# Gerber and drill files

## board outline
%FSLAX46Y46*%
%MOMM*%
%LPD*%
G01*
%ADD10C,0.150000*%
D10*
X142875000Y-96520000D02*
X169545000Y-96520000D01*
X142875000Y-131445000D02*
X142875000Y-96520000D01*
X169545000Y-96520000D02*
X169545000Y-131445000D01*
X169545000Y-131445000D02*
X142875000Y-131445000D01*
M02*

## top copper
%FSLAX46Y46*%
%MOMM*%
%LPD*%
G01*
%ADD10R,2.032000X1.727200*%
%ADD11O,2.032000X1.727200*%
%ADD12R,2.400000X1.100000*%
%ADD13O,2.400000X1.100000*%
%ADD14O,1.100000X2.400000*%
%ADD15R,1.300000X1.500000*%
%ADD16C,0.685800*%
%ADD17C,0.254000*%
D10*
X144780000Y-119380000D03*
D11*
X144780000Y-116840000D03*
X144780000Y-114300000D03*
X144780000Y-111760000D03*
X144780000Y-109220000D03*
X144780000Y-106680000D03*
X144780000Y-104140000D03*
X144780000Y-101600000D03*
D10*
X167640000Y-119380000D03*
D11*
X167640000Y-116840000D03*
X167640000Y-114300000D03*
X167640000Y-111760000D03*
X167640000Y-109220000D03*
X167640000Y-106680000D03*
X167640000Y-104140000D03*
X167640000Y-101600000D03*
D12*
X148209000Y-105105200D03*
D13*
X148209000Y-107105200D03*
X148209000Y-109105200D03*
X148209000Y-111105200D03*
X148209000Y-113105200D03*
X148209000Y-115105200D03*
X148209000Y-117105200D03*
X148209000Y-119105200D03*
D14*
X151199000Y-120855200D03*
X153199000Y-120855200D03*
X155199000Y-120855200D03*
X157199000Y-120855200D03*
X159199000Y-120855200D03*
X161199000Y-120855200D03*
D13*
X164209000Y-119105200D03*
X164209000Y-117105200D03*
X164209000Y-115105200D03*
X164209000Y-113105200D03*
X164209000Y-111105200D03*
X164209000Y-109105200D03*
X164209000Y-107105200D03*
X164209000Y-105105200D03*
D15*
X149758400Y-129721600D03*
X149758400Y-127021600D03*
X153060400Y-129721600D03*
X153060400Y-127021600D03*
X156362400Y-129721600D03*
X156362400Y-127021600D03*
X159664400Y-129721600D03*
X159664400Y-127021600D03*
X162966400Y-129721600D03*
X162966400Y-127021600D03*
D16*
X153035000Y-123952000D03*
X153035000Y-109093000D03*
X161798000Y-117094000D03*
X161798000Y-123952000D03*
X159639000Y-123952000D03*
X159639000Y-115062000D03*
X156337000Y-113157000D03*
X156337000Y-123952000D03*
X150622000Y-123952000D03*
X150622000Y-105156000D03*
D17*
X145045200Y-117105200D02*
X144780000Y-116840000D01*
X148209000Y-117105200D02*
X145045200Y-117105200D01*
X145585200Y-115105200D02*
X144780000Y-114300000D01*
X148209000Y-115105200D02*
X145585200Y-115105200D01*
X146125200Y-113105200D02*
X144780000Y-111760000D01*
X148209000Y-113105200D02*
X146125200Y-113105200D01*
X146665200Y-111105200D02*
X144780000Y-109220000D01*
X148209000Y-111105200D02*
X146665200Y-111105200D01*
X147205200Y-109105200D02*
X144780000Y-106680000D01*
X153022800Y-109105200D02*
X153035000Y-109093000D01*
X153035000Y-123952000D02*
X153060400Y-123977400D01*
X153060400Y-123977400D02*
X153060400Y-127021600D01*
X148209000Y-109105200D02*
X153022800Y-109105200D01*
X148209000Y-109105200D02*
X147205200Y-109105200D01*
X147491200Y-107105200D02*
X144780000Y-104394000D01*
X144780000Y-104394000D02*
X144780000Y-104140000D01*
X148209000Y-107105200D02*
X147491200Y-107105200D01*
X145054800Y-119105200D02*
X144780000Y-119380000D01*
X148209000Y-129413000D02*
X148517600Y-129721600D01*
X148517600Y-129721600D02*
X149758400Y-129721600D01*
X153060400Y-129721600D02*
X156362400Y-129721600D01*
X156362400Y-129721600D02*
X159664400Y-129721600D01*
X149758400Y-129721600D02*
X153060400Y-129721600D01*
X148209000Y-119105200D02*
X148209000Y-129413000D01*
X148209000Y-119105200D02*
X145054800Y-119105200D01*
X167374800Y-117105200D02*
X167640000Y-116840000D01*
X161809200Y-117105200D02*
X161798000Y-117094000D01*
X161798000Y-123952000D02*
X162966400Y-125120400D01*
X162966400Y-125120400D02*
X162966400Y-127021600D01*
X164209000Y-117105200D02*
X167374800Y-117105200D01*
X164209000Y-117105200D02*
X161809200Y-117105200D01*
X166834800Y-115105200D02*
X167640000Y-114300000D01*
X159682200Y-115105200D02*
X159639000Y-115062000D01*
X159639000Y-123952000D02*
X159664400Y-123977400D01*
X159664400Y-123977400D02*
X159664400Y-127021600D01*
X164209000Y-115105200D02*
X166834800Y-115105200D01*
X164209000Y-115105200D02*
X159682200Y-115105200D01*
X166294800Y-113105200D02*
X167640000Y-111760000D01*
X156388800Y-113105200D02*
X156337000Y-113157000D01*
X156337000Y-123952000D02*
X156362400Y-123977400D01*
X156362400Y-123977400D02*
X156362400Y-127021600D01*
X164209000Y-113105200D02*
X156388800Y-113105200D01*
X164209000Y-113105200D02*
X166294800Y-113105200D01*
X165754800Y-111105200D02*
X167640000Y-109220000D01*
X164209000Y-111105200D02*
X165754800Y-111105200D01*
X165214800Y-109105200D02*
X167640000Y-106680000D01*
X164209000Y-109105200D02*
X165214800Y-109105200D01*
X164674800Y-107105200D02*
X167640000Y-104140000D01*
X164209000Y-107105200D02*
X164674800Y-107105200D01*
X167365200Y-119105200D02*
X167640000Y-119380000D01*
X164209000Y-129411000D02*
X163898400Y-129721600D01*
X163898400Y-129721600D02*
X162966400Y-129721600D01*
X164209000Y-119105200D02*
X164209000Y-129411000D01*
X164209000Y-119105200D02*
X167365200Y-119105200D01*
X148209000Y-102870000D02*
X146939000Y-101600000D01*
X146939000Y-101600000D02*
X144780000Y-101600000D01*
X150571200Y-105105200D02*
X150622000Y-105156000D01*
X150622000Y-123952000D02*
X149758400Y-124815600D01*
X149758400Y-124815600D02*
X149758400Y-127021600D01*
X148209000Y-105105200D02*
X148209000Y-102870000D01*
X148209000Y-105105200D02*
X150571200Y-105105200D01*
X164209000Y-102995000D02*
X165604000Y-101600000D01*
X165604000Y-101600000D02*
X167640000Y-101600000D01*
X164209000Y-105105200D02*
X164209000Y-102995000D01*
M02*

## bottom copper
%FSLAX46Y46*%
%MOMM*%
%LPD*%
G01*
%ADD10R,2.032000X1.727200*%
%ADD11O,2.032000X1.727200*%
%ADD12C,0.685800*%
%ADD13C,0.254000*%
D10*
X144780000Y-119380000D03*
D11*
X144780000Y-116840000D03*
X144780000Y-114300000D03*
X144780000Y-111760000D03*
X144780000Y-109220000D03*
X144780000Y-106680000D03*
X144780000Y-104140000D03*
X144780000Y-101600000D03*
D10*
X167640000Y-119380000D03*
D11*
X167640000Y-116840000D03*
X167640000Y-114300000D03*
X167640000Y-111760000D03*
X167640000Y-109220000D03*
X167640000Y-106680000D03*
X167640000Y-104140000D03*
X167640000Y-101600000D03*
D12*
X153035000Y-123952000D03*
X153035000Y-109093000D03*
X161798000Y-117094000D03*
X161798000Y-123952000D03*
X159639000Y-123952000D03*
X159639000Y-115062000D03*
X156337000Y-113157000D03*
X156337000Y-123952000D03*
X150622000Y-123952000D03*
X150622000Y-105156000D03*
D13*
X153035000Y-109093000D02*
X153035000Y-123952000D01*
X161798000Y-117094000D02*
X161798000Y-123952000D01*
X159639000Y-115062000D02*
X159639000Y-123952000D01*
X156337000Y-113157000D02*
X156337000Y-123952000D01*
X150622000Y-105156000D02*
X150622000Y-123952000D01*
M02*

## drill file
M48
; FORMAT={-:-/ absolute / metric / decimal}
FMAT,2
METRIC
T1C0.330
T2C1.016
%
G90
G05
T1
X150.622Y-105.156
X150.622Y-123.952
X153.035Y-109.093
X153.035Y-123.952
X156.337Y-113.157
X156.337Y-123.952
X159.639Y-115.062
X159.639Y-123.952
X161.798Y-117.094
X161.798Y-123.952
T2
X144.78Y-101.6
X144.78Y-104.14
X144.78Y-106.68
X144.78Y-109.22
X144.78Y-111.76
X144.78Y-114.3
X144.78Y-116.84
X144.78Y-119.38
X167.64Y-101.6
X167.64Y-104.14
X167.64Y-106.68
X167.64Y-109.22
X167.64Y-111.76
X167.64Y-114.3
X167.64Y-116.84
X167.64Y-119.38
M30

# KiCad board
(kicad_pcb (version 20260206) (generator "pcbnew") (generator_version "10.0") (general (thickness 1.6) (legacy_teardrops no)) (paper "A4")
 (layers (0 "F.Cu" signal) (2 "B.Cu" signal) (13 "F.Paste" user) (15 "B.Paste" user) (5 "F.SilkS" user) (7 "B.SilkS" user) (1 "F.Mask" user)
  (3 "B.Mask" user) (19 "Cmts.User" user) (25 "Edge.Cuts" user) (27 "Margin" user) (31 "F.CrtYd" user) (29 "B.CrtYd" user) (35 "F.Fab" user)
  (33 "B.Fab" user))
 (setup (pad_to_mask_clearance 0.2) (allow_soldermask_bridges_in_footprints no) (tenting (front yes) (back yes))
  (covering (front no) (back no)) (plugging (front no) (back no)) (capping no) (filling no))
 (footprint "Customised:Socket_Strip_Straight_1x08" (layer "F.Cu") (at 144.78 119.38 90)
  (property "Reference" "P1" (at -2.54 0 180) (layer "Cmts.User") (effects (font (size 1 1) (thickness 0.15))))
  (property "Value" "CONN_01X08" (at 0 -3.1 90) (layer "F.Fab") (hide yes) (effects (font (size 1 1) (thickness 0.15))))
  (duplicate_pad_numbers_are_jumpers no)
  (pad "1" thru_hole rect (at 0 0 90) (size 1.7272 2.032) (drill 1.016) (layers "*.Cu" "*.Mask") (remove_unused_layers no) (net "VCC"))
  (pad "2" thru_hole oval (at 2.54 0 90) (size 1.7272 2.032) (drill 1.016) (layers "*.Cu" "*.Mask") (remove_unused_layers no)
   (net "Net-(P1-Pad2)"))
  (pad "3" thru_hole oval (at 5.08 0 90) (size 1.7272 2.032) (drill 1.016) (layers "*.Cu" "*.Mask") (remove_unused_layers no)
   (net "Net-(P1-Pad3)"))
  (pad "4" thru_hole oval (at 7.62 0 90) (size 1.7272 2.032) (drill 1.016) (layers "*.Cu" "*.Mask") (remove_unused_layers no)
   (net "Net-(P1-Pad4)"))
  (pad "5" thru_hole oval (at 10.16 0 90) (size 1.7272 2.032) (drill 1.016) (layers "*.Cu" "*.Mask") (remove_unused_layers no)
   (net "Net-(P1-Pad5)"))
  (pad "6" thru_hole oval (at 12.7 0 90) (size 1.7272 2.032) (drill 1.016) (layers "*.Cu" "*.Mask") (remove_unused_layers no)
   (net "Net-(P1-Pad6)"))
  (pad "7" thru_hole oval (at 15.24 0 90) (size 1.7272 2.032) (drill 1.016) (layers "*.Cu" "*.Mask") (remove_unused_layers no)
   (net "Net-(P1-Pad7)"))
  (pad "8" thru_hole oval (at 17.78 0 90) (size 1.7272 2.032) (drill 1.016) (layers "*.Cu" "*.Mask") (remove_unused_layers no)
   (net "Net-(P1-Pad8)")))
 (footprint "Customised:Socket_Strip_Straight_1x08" (layer "F.Cu") (at 167.64 119.38 90)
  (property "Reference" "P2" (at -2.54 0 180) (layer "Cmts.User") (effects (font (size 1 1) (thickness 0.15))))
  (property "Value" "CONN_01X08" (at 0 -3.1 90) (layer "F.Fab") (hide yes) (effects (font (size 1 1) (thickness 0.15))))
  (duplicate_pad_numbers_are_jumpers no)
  (pad "1" thru_hole rect (at 0 0 90) (size 1.7272 2.032) (drill 1.016) (layers "*.Cu" "*.Mask") (remove_unused_layers no) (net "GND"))
  (pad "2" thru_hole oval (at 2.54 0 90) (size 1.7272 2.032) (drill 1.016) (layers "*.Cu" "*.Mask") (remove_unused_layers no)
   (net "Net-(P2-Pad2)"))
  (pad "3" thru_hole oval (at 5.08 0 90) (size 1.7272 2.032) (drill 1.016) (layers "*.Cu" "*.Mask") (remove_unused_layers no)
   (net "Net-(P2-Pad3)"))
  (pad "4" thru_hole oval (at 7.62 0 90) (size 1.7272 2.032) (drill 1.016) (layers "*.Cu" "*.Mask") (remove_unused_layers no)
   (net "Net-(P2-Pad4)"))
  (pad "5" thru_hole oval (at 10.16 0 90) (size 1.7272 2.032) (drill 1.016) (layers "*.Cu" "*.Mask") (remove_unused_layers no)
   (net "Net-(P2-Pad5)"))
  (pad "6" thru_hole oval (at 12.7 0 90) (size 1.7272 2.032) (drill 1.016) (layers "*.Cu" "*.Mask") (remove_unused_layers no)
   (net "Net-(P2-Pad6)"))
  (pad "7" thru_hole oval (at 15.24 0 90) (size 1.7272 2.032) (drill 1.016) (layers "*.Cu" "*.Mask") (remove_unused_layers no)
   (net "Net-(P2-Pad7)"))
  (pad "8" thru_hole oval (at 17.78 0 90) (size 1.7272 2.032) (drill 1.016) (layers "*.Cu" "*.Mask") (remove_unused_layers no)
   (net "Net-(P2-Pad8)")))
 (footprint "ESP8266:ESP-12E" (layer "F.Cu") (at 148.209 105.1052)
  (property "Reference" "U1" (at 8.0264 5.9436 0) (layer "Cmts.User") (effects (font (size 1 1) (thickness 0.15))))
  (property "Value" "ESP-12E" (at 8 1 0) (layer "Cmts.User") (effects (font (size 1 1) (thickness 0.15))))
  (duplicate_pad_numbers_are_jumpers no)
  (pad "1" smd rect (at 0 0) (size 2.4 1.1) (layers "F.Cu" "F.Mask" "F.Paste") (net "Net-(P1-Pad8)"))
  (pad "2" smd oval (at 0 2) (size 2.4 1.1) (layers "F.Cu" "F.Mask" "F.Paste") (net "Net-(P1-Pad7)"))
  (pad "3" smd oval (at 0 4) (size 2.4 1.1) (layers "F.Cu" "F.Mask" "F.Paste") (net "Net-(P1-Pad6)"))
  (pad "4" smd oval (at 0 6) (size 2.4 1.1) (layers "F.Cu" "F.Mask" "F.Paste") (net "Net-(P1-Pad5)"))
  (pad "5" smd oval (at 0 8) (size 2.4 1.1) (layers "F.Cu" "F.Mask" "F.Paste") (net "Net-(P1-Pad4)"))
  (pad "6" smd oval (at 0 10) (size 2.4 1.1) (layers "F.Cu" "F.Mask" "F.Paste") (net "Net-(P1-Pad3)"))
  (pad "7" smd oval (at 0 12) (size 2.4 1.1) (layers "F.Cu" "F.Mask" "F.Paste") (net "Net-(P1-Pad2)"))
  (pad "8" smd oval (at 0 14) (size 2.4 1.1) (layers "F.Cu" "F.Mask" "F.Paste") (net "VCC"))
  (pad "9" smd oval (at 2.99 15.75 90) (size 2.4 1.1) (layers "F.Cu" "F.Mask" "F.Paste") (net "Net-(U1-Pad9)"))
  (pad "10" smd oval (at 4.99 15.75 90) (size 2.4 1.1) (layers "F.Cu" "F.Mask" "F.Paste") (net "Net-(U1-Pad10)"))
  (pad "11" smd oval (at 6.99 15.75 90) (size 2.4 1.1) (layers "F.Cu" "F.Mask" "F.Paste") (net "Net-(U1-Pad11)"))
  (pad "12" smd oval (at 8.99 15.75 90) (size 2.4 1.1) (layers "F.Cu" "F.Mask" "F.Paste") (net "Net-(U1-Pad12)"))
  (pad "13" smd oval (at 10.99 15.75 90) (size 2.4 1.1) (layers "F.Cu" "F.Mask" "F.Paste") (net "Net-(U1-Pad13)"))
  (pad "14" smd oval (at 12.99 15.75 90) (size 2.4 1.1) (layers "F.Cu" "F.Mask" "F.Paste") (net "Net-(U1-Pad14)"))
  (pad "15" smd oval (at 16 14) (size 2.4 1.1) (layers "F.Cu" "F.Mask" "F.Paste") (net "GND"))
  (pad "16" smd oval (at 16 12) (size 2.4 1.1) (layers "F.Cu" "F.Mask" "F.Paste") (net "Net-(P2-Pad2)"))
  (pad "17" smd oval (at 16 10) (size 2.4 1.1) (layers "F.Cu" "F.Mask" "F.Paste") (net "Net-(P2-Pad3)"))
  (pad "18" smd oval (at 16 8) (size 2.4 1.1) (layers "F.Cu" "F.Mask" "F.Paste") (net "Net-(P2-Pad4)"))
  (pad "19" smd oval (at 16 6) (size 2.4 1.1) (layers "F.Cu" "F.Mask" "F.Paste") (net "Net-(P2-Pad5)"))
  (pad "20" smd oval (at 16 4) (size 2.4 1.1) (layers "F.Cu" "F.Mask" "F.Paste") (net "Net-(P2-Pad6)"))
  (pad "21" smd oval (at 16 2) (size 2.4 1.1) (layers "F.Cu" "F.Mask" "F.Paste") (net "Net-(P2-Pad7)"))
  (pad "22" smd oval (at 16 0) (size 2.4 1.1) (layers "F.Cu" "F.Mask" "F.Paste") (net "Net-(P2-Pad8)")))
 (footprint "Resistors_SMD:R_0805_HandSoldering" (layer "F.Cu") (at 149.7584 128.3716 90)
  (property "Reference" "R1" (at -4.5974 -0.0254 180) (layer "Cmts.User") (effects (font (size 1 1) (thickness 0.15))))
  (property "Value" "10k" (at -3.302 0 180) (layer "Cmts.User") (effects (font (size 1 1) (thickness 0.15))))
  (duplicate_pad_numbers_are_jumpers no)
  (pad "1" smd rect (at -1.35 0 90) (size 1.5 1.3) (layers "F.Cu" "F.Mask" "F.Paste") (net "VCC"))
  (pad "2" smd rect (at 1.35 0 90) (size 1.5 1.3) (layers "F.Cu" "F.Mask" "F.Paste") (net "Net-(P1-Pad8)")))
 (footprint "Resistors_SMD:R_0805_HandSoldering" (layer "F.Cu") (at 153.0604 128.3716 90)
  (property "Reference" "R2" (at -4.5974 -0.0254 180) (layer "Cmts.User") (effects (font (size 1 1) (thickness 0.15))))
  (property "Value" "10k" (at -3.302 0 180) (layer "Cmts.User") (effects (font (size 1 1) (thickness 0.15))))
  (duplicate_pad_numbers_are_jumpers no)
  (pad "1" smd rect (at -1.35 0 90) (size 1.5 1.3) (layers "F.Cu" "F.Mask" "F.Paste") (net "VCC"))
  (pad "2" smd rect (at 1.35 0 90) (size 1.5 1.3) (layers "F.Cu" "F.Mask" "F.Paste") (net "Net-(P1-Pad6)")))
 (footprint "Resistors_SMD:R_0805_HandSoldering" (layer "F.Cu") (at 156.3624 128.3716 90)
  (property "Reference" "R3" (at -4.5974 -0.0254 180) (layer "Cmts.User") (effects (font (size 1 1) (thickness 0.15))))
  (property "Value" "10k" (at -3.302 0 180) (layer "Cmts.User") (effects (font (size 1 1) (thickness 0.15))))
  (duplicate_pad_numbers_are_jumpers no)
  (pad "1" smd rect (at -1.35 0 90) (size 1.5 1.3) (layers "F.Cu" "F.Mask" "F.Paste") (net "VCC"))
  (pad "2" smd rect (at 1.35 0 90) (size 1.5 1.3) (layers "F.Cu" "F.Mask" "F.Paste") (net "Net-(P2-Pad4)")))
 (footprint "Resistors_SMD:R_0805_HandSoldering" (layer "F.Cu") (at 159.6644 128.3716 90)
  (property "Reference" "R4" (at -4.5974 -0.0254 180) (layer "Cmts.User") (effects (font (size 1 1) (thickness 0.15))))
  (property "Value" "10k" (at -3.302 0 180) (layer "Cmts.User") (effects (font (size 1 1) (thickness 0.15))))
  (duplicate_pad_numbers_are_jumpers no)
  (pad "1" smd rect (at -1.35 0 90) (size 1.5 1.3) (layers "F.Cu" "F.Mask" "F.Paste") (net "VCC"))
  (pad "2" smd rect (at 1.35 0 90) (size 1.5 1.3) (layers "F.Cu" "F.Mask" "F.Paste") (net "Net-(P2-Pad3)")))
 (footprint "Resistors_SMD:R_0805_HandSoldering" (layer "F.Cu") (at 162.9664 128.3716 90)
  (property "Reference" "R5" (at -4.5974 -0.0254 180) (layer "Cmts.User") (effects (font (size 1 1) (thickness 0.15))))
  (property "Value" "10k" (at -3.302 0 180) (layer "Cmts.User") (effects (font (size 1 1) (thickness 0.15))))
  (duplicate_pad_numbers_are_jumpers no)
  (pad "1" smd rect (at -1.35 0 90) (size 1.5 1.3) (layers "F.Cu" "F.Mask" "F.Paste") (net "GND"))
  (pad "2" smd rect (at 1.35 0 90) (size 1.5 1.3) (layers "F.Cu" "F.Mask" "F.Paste") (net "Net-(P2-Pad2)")))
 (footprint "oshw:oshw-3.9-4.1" (layer "F.Cu") (at 167.005 128.27)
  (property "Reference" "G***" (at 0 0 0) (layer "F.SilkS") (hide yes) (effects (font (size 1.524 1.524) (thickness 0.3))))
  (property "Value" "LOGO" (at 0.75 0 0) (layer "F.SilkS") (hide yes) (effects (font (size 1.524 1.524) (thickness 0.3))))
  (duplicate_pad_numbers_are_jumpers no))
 (gr_line (start 142.875 96.52) (end 169.545 96.52) (stroke (width 0.15) (type solid)) (layer "Edge.Cuts"))
 (gr_line (start 142.875 131.445) (end 142.875 96.52) (stroke (width 0.15) (type solid)) (layer "Edge.Cuts"))
 (gr_line (start 169.545 96.52) (end 169.545 131.445) (stroke (width 0.15) (type solid)) (layer "Edge.Cuts"))
 (gr_line (start 169.545 131.445) (end 142.875 131.445) (stroke (width 0.15) (type solid)) (layer "Edge.Cuts"))
 (segment (start 145.0452 117.1052) (end 144.78 116.84) (width 0.254) (layer "F.Cu") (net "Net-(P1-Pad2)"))
 (segment (start 148.209 117.1052) (end 145.0452 117.1052) (width 0.254) (layer "F.Cu") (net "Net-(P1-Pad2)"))
 (segment (start 145.5852 115.1052) (end 144.78 114.3) (width 0.254) (layer "F.Cu") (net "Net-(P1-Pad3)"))
 (segment (start 148.209 115.1052) (end 145.5852 115.1052) (width 0.254) (layer "F.Cu") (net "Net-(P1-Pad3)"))
 (segment (start 146.1252 113.1052) (end 144.78 111.76) (width 0.254) (layer "F.Cu") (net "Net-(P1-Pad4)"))
 (segment (start 148.209 113.1052) (end 146.1252 113.1052) (width 0.254) (layer "F.Cu") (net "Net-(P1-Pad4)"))
 (segment (start 146.6652 111.1052) (end 144.78 109.22) (width 0.254) (layer "F.Cu") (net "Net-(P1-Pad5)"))
 (segment (start 148.209 111.1052) (end 146.6652 111.1052) (width 0.254) (layer "F.Cu") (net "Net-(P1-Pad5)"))
 (segment (start 147.2052 109.1052) (end 144.78 106.68) (width 0.254) (layer "F.Cu") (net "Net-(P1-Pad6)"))
 (segment (start 153.0228 109.1052) (end 153.035 109.093) (width 0.254) (layer "F.Cu") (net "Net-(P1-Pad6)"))
 (segment (start 153.035 123.952) (end 153.0604 123.9774) (width 0.254) (layer "F.Cu") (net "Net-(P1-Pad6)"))
 (segment (start 153.0604 123.9774) (end 153.0604 127.0216) (width 0.254) (layer "F.Cu") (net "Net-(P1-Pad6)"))
 (segment (start 148.209 109.1052) (end 153.0228 109.1052) (width 0.254) (layer "F.Cu") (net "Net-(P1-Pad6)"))
 (segment (start 148.209 109.1052) (end 147.2052 109.1052) (width 0.254) (layer "F.Cu") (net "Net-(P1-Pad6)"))
 (via (at 153.035 123.952) (size 0.6858) (drill 0.3302) (layers "F.Cu" "B.Cu") (capping no) (covering (front no) (back no))
  (plugging (front no) (back no)) (filling no) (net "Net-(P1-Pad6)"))
 (via (at 153.035 109.093) (size 0.6858) (drill 0.3302) (layers "F.Cu" "B.Cu") (capping no) (covering (front no) (back no))
  (plugging (front no) (back no)) (filling no) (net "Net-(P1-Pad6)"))
 (segment (start 153.035 109.093) (end 153.035 123.952) (width 0.254) (layer "B.Cu") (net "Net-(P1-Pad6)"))
 (segment (start 147.4912 107.1052) (end 144.78 104.394) (width 0.254) (layer "F.Cu") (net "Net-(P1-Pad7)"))
 (segment (start 144.78 104.394) (end 144.78 104.14) (width 0.254) (layer "F.Cu") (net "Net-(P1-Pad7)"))
 (segment (start 148.209 107.1052) (end 147.4912 107.1052) (width 0.254) (layer "F.Cu") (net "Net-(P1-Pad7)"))
 (segment (start 145.0548 119.1052) (end 144.78 119.38) (width 0.254) (layer "F.Cu") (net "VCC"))
 (segment (start 148.209 129.413) (end 148.5176 129.7216) (width 0.254) (layer "F.Cu") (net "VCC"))
 (segment (start 148.5176 129.7216) (end 149.7584 129.7216) (width 0.254) (layer "F.Cu") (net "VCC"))
 (segment (start 153.0604 129.7216) (end 156.3624 129.7216) (width 0.254) (layer "F.Cu") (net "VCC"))
 (segment (start 156.3624 129.7216) (end 159.6644 129.7216) (width 0.254) (layer "F.Cu") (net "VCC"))
 (segment (start 149.7584 129.7216) (end 153.0604 129.7216) (width 0.254) (layer "F.Cu") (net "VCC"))
 (segment (start 148.209 119.1052) (end 148.209 129.413) (width 0.254) (layer "F.Cu") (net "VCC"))
 (segment (start 148.209 119.1052) (end 145.0548 119.1052) (width 0.254) (layer "F.Cu") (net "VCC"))
 (segment (start 167.3748 117.1052) (end 167.64 116.84) (width 0.254) (layer "F.Cu") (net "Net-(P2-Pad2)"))
 (segment (start 161.8092 117.1052) (end 161.798 117.094) (width 0.254) (layer "F.Cu") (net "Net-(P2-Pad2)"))
 (segment (start 161.798 123.952) (end 162.9664 125.1204) (width 0.254) (layer "F.Cu") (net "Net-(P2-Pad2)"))
 (segment (start 162.9664 125.1204) (end 162.9664 127.0216) (width 0.254) (layer "F.Cu") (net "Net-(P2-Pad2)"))
 (segment (start 164.209 117.1052) (end 167.3748 117.1052) (width 0.254) (layer "F.Cu") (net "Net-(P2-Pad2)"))
 (segment (start 164.209 117.1052) (end 161.8092 117.1052) (width 0.254) (layer "F.Cu") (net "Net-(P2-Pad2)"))
 (via (at 161.798 117.094) (size 0.6858) (drill 0.3302) (layers "F.Cu" "B.Cu") (capping no) (covering (front no) (back no))
  (plugging (front no) (back no)) (filling no) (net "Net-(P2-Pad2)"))
 (via (at 161.798 123.952) (size 0.6858) (drill 0.3302) (layers "F.Cu" "B.Cu") (capping no) (covering (front no) (back no))
  (plugging (front no) (back no)) (filling no) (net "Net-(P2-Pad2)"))
 (segment (start 161.798 117.094) (end 161.798 123.952) (width 0.254) (layer "B.Cu") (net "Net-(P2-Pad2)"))
 (segment (start 166.8348 115.1052) (end 167.64 114.3) (width 0.254) (layer "F.Cu") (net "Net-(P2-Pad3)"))
 (segment (start 159.6822 115.1052) (end 159.639 115.062) (width 0.254) (layer "F.Cu") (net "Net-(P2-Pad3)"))
 (segment (start 159.639 123.952) (end 159.6644 123.9774) (width 0.254) (layer "F.Cu") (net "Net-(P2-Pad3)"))
 (segment (start 159.6644 123.9774) (end 159.6644 127.0216) (width 0.254) (layer "F.Cu") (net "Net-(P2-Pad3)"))
 (segment (start 164.209 115.1052) (end 166.8348 115.1052) (width 0.254) (layer "F.Cu") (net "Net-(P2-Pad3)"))
 (segment (start 164.209 115.1052) (end 159.6822 115.1052) (width 0.254) (layer "F.Cu") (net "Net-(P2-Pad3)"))
 (via (at 159.639 123.952) (size 0.6858) (drill 0.3302) (layers "F.Cu" "B.Cu") (capping no) (covering (front no) (back no))
  (plugging (front no) (back no)) (filling no) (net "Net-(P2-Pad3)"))
 (via (at 159.639 115.062) (size 0.6858) (drill 0.3302) (layers "F.Cu" "B.Cu") (capping no) (covering (front no) (back no))
  (plugging (front no) (back no)) (filling no) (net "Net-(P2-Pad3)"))
 (segment (start 159.639 115.062) (end 159.639 123.952) (width 0.254) (layer "B.Cu") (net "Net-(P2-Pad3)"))
 (segment (start 166.2948 113.1052) (end 167.64 111.76) (width 0.254) (layer "F.Cu") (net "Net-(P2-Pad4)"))
 (segment (start 156.3888 113.1052) (end 156.337 113.157) (width 0.254) (layer "F.Cu") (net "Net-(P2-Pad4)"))
 (segment (start 156.337 123.952) (end 156.3624 123.9774) (width 0.254) (layer "F.Cu") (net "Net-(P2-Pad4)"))
 (segment (start 156.3624 123.9774) (end 156.3624 127.0216) (width 0.254) (layer "F.Cu") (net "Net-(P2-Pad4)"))
 (segment (start 164.209 113.1052) (end 156.3888 113.1052) (width 0.254) (layer "F.Cu") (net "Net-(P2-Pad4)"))
 (segment (start 164.209 113.1052) (end 166.2948 113.1052) (width 0.254) (layer "F.Cu") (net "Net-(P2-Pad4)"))
 (via (at 156.337 113.157) (size 0.6858) (drill 0.3302) (layers "F.Cu" "B.Cu") (capping no) (covering (front no) (back no))
  (plugging (front no) (back no)) (filling no) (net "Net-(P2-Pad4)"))
 (via (at 156.337 123.952) (size 0.6858) (drill 0.3302) (layers "F.Cu" "B.Cu") (capping no) (covering (front no) (back no))
  (plugging (front no) (back no)) (filling no) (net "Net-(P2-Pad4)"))
 (segment (start 156.337 113.157) (end 156.337 123.952) (width 0.254) (layer "B.Cu") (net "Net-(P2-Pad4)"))
 (segment (start 165.7548 111.1052) (end 167.64 109.22) (width 0.254) (layer "F.Cu") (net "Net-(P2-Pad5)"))
 (segment (start 164.209 111.1052) (end 165.7548 111.1052) (width 0.254) (layer "F.Cu") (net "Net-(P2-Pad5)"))
 (segment (start 165.2148 109.1052) (end 167.64 106.68) (width 0.254) (layer "F.Cu") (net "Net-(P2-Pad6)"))
 (segment (start 164.209 109.1052) (end 165.2148 109.1052) (width 0.254) (layer "F.Cu") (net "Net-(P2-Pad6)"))
 (segment (start 164.6748 107.1052) (end 167.64 104.14) (width 0.254) (layer "F.Cu") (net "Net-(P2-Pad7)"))
 (segment (start 164.209 107.1052) (end 164.6748 107.1052) (width 0.254) (layer "F.Cu") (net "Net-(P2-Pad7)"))
 (segment (start 167.3652 119.1052) (end 167.64 119.38) (width 0.254) (layer "F.Cu") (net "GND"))
 (segment (start 164.209 129.411) (end 163.8984 129.7216) (width 0.254) (layer "F.Cu") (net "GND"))
 (segment (start 163.8984 129.7216) (end 162.9664 129.7216) (width 0.254) (layer "F.Cu") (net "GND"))
 (segment (start 164.209 119.1052) (end 164.209 129.411) (width 0.254) (layer "F.Cu") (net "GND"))
 (segment (start 164.209 119.1052) (end 167.3652 119.1052) (width 0.254) (layer "F.Cu") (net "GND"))
 (segment (start 148.209 102.87) (end 146.939 101.6) (width 0.254) (layer "F.Cu") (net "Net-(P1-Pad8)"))
 (segment (start 146.939 101.6) (end 144.78 101.6) (width 0.254) (layer "F.Cu") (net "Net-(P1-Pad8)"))
 (segment (start 150.5712 105.1052) (end 150.622 105.156) (width 0.254) (layer "F.Cu") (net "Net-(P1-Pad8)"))
 (segment (start 150.622 123.952) (end 149.7584 124.8156) (width 0.254) (layer "F.Cu") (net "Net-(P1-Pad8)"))
 (segment (start 149.7584 124.8156) (end 149.7584 127.0216) (width 0.254) (layer "F.Cu") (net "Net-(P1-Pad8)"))
 (segment (start 148.209 105.1052) (end 148.209 102.87) (width 0.254) (layer "F.Cu") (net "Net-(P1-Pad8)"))
 (segment (start 148.209 105.1052) (end 150.5712 105.1052) (width 0.254) (layer "F.Cu") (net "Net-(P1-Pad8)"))
 (via (at 150.622 123.952) (size 0.6858) (drill 0.3302) (layers "F.Cu" "B.Cu") (capping no) (covering (front no) (back no))
  (plugging (front no) (back no)) (filling no) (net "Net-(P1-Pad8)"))
 (via (at 150.622 105.156) (size 0.6858) (drill 0.3302) (layers "F.Cu" "B.Cu") (capping no) (covering (front no) (back no))
  (plugging (front no) (back no)) (filling no) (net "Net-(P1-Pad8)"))
 (segment (start 150.622 105.156) (end 150.622 123.952) (width 0.254) (layer "B.Cu") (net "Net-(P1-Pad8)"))
 (segment (start 164.209 102.995) (end 165.604 101.6) (width 0.254) (layer "F.Cu") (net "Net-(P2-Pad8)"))
 (segment (start 165.604 101.6) (end 167.64 101.6) (width 0.254) (layer "F.Cu") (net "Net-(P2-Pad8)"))
 (segment (start 164.209 105.1052) (end 164.209 102.995) (width 0.254) (layer "F.Cu") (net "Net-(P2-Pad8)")))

